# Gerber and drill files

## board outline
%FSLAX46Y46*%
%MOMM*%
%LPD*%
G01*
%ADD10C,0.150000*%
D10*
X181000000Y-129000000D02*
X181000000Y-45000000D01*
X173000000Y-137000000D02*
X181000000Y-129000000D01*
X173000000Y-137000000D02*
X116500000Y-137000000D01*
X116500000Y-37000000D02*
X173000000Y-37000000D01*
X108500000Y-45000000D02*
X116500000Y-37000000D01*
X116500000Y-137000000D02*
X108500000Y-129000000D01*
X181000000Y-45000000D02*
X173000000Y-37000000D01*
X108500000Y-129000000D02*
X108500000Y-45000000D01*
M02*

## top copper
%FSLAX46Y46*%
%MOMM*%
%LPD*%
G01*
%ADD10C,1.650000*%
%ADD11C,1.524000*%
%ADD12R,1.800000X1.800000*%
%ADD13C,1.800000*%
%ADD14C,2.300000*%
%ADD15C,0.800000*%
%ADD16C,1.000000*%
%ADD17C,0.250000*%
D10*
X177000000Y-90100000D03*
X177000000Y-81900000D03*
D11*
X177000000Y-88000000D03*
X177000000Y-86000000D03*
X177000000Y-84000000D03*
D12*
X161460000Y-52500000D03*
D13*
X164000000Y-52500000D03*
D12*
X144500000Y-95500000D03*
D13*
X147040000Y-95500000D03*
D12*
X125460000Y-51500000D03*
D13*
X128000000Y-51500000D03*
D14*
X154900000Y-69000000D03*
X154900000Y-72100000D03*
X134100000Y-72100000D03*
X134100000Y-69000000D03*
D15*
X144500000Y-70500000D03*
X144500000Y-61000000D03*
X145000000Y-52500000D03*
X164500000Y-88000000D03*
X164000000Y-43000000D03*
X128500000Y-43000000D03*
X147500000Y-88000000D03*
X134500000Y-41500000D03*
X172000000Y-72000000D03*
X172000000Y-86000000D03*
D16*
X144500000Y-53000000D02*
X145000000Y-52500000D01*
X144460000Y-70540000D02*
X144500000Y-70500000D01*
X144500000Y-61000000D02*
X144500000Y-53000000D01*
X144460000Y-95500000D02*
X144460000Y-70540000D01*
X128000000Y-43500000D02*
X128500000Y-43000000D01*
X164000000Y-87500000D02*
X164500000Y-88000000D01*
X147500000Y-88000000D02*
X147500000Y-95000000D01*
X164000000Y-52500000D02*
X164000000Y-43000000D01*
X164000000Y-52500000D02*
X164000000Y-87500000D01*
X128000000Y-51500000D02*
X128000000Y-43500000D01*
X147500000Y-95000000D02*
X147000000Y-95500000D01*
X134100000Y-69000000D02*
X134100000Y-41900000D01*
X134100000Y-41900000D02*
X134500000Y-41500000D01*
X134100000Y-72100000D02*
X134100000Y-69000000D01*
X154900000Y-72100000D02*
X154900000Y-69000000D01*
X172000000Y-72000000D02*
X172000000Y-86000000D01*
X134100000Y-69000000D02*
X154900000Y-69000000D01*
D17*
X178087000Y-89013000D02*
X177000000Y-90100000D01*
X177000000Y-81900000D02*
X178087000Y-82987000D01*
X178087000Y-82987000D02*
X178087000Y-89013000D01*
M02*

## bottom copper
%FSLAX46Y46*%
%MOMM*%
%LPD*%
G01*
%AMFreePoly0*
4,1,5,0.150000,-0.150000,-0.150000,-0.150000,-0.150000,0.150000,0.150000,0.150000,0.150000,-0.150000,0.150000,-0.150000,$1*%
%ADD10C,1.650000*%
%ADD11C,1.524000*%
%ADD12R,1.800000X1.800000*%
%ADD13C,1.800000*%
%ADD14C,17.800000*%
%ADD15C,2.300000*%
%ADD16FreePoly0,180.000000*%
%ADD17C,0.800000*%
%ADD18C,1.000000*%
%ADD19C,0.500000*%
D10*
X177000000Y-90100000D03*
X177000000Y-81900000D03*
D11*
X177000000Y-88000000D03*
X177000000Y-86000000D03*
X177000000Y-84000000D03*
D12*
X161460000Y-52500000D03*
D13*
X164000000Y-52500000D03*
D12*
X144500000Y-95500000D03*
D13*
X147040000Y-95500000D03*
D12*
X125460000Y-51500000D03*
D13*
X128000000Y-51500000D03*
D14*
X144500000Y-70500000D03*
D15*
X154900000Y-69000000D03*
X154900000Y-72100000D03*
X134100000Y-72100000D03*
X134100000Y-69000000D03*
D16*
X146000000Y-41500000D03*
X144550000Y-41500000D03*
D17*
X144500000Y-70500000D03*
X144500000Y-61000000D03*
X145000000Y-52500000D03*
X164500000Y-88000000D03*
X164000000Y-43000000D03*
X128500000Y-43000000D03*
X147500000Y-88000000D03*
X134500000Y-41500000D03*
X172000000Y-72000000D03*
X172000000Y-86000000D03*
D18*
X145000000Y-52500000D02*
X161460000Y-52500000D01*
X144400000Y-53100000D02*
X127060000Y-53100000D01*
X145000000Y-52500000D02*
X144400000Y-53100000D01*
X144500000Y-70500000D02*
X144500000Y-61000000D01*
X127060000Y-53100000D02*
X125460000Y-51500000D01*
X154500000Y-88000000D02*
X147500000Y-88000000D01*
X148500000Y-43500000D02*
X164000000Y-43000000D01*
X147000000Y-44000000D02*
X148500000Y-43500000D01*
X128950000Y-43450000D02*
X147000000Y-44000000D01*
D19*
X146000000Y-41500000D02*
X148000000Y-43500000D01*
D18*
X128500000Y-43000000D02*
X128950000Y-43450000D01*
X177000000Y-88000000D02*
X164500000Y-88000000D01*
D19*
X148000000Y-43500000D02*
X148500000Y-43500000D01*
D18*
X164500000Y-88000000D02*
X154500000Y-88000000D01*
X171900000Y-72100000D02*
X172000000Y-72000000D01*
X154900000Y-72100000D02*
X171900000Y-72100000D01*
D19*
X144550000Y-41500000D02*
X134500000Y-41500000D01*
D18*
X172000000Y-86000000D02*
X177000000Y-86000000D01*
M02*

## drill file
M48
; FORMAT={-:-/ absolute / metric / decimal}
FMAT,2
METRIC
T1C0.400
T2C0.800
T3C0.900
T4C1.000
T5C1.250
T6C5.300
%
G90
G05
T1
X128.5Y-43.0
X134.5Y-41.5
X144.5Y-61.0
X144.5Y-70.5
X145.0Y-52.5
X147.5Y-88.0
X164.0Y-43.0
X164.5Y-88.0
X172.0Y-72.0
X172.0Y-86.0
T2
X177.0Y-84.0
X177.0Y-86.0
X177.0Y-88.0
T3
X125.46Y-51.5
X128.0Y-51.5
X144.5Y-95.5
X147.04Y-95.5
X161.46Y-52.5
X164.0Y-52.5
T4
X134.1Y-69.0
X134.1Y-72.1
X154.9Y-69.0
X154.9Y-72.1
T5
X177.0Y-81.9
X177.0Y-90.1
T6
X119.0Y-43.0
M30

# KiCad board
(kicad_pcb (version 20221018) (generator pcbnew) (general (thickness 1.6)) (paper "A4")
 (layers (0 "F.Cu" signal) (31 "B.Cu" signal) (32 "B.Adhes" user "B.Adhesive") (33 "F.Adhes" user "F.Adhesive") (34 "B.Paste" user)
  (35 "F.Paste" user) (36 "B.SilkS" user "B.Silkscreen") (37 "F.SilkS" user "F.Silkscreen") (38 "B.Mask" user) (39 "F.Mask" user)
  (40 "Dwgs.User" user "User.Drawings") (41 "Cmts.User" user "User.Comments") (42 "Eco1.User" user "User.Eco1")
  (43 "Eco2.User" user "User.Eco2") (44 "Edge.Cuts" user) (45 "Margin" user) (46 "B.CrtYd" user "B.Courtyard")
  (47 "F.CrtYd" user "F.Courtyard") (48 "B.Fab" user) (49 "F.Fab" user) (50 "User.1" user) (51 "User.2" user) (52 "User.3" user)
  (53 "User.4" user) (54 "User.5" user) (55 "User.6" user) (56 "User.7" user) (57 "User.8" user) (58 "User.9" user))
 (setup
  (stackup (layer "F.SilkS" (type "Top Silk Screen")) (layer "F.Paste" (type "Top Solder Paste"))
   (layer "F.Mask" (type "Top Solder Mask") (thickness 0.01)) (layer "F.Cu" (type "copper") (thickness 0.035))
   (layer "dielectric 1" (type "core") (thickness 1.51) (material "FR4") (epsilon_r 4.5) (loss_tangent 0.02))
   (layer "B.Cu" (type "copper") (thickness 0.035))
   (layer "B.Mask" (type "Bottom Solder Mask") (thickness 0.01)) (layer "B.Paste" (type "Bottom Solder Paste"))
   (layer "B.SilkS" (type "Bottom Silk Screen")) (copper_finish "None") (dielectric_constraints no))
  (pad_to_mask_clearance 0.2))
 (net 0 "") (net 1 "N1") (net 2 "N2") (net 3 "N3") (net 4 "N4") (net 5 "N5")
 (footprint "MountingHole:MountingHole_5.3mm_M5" (layer "F.Cu") (at 119 43)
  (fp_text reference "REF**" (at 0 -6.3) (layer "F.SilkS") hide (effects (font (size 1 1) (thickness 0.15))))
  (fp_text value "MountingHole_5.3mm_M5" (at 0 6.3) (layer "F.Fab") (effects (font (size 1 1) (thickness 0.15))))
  (pad "" np_thru_hole circle (at 0 0) (size 5.3 5.3) (drill 5.3) (layers "*.Cu" "*.Mask")))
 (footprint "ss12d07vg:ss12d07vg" (layer "F.Cu") (at 177 90.1 90)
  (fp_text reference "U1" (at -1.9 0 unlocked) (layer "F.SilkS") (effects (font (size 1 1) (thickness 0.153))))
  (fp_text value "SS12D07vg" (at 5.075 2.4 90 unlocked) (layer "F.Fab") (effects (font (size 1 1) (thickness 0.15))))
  (pad "1" thru_hole circle (at 0 0 90) (size 1.65 1.65) (drill 1.25) (layers "*.Cu" "*.Mask") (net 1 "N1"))
  (pad "1" thru_hole circle (at 8.2 0 90) (size 1.65 1.65) (drill 1.25) (layers "*.Cu" "*.Mask") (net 1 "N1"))
  (pad "2" thru_hole circle (at 2.1 0 90) (size 1.524 1.524) (drill 0.8) (layers "*.Cu" "*.Mask") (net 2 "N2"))
  (pad "3" thru_hole circle (at 4.1 0 90) (size 1.524 1.524) (drill 0.8) (layers "*.Cu" "*.Mask") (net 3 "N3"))
  (pad "4" thru_hole circle (at 6.1 0 90) (size 1.524 1.524) (drill 0.8) (layers "*.Cu" "*.Mask") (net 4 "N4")))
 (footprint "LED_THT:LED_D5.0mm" (layer "F.Cu") (at 161.46 52.5)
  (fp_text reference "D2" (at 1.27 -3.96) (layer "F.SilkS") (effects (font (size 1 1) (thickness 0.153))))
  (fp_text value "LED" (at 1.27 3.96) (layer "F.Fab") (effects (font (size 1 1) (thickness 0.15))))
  (pad "1" thru_hole rect (at 0 0) (size 1.8 1.8) (drill 0.9) (layers "*.Cu" "*.Mask") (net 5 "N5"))
  (pad "2" thru_hole circle (at 2.54 0) (size 1.8 1.8) (drill 0.9) (layers "*.Cu" "*.Mask") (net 2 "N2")))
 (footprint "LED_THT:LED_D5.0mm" (layer "F.Cu") (at 144.5 95.5)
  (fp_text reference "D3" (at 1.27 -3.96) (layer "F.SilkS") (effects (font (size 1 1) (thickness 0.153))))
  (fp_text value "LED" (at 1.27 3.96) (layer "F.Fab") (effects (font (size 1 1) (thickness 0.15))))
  (pad "1" thru_hole rect (at 0 0) (size 1.8 1.8) (drill 0.9) (layers "*.Cu" "*.Mask") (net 5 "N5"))
  (pad "2" thru_hole circle (at 2.54 0) (size 1.8 1.8) (drill 0.9) (layers "*.Cu" "*.Mask") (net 2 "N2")))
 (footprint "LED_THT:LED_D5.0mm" (layer "F.Cu") (at 125.46 51.5)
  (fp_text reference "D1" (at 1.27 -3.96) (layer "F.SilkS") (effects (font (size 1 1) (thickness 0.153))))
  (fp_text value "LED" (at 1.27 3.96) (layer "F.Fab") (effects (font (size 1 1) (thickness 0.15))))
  (pad "1" thru_hole rect (at 0 0) (size 1.8 1.8) (drill 0.9) (layers "*.Cu" "*.Mask") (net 5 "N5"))
  (pad "2" thru_hole circle (at 2.54 0) (size 1.8 1.8) (drill 0.9) (layers "*.Cu" "*.Mask") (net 2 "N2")))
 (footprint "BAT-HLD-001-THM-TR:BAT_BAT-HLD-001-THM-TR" (layer "B.Cu") (at 144.5 70.5 180)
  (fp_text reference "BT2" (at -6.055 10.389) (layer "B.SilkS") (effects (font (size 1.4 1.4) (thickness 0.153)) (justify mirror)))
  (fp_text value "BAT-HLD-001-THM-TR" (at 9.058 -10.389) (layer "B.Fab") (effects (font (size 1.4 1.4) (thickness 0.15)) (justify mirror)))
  (pad "N" smd circle (at 0 0 180) (size 17.8 17.8) (layers "B.Cu" "B.Mask") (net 5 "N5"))
  (pad "P1" thru_hole circle (at -10.4 1.5 180) (size 2.3 2.3) (drill 1) (layers "*.Cu" "*.Mask") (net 3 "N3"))
  (pad "P2" thru_hole circle (at -10.4 -1.6 180) (size 2.3 2.3) (drill 1) (layers "*.Cu" "*.Mask") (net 3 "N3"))
  (pad "P3" thru_hole circle (at 10.4 -1.6 180) (size 2.3 2.3) (drill 1) (layers "*.Cu" "*.Mask") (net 3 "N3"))
  (pad "P4" thru_hole circle (at 10.4 1.5 180) (size 2.3 2.3) (drill 1) (layers "*.Cu" "*.Mask") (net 3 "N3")))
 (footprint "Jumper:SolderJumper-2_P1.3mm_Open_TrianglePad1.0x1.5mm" (layer "B.Cu") (at 145.275 41.5 180)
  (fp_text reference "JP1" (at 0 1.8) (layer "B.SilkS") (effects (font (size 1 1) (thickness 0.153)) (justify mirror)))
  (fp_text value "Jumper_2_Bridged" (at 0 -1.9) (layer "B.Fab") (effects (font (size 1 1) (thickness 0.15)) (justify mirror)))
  (pad "1" smd custom (at -0.725 0 180) (size 0.3 0.3) (layers "B.Cu" "B.Mask") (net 2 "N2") (zone_connect 2) (thermal_bridge_angle 45)
   (options (clearance outline) (anchor rect)) (primitives))
  (pad "2" smd custom (at 0.725 0 180) (size 0.3 0.3) (layers "B.Cu" "B.Mask") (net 3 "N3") (zone_connect 2) (thermal_bridge_angle 45)
   (options (clearance outline) (anchor rect)) (primitives)))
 (gr_line (start 181 129) (end 181 45) (stroke (width 0.15) (type default)) (layer "Edge.Cuts"))
 (gr_line (start 173 137) (end 181 129) (stroke (width 0.15) (type default)) (layer "Edge.Cuts"))
 (gr_line (start 173 137) (end 116.5 137) (stroke (width 0.15) (type default)) (layer "Edge.Cuts"))
 (gr_line (start 116.5 37) (end 173 37) (stroke (width 0.15) (type default)) (layer "Edge.Cuts"))
 (gr_line (start 108.5 45) (end 116.5 37) (stroke (width 0.15) (type default)) (layer "Edge.Cuts"))
 (gr_line (start 116.5 137) (end 108.5 129) (stroke (width 0.15) (type default)) (layer "Edge.Cuts"))
 (gr_line (start 181 45) (end 173 37) (stroke (width 0.15) (type default)) (layer "Edge.Cuts"))
 (gr_line (start 108.5 129) (end 108.5 45) (stroke (width 0.15) (type default)) (layer "Edge.Cuts"))
 (segment (start 144.5 53) (end 145 52.5) (width 1) (layer "F.Cu") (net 5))
 (segment (start 144.46 70.54) (end 144.5 70.5) (width 1) (layer "F.Cu") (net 5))
 (segment (start 144.5 61) (end 144.5 53) (width 1) (layer "F.Cu") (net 5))
 (segment (start 144.46 95.5) (end 144.46 70.54) (width 1) (layer "F.Cu") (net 5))
 (via (at 144.5 70.5) (size 0.8) (drill 0.4) (layers "F.Cu" "B.Cu") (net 5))
 (via (at 144.5 61) (size 0.8) (drill 0.4) (layers "F.Cu" "B.Cu") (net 5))
 (via (at 145 52.5) (size 0.8) (drill 0.4) (layers "F.Cu" "B.Cu") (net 5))
 (segment (start 145 52.5) (end 161.46 52.5) (width 1) (layer "B.Cu") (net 5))
 (segment (start 144.4 53.1) (end 127.06 53.1) (width 1) (layer "B.Cu") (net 5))
 (segment (start 145 52.5) (end 144.4 53.1) (width 1) (layer "B.Cu") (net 5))
 (segment (start 144.5 70.5) (end 144.5 61) (width 1) (layer "B.Cu") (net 5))
 (segment (start 127.06 53.1) (end 125.46 51.5) (width 1) (layer "B.Cu") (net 5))
 (segment (start 128 43.5) (end 128.5 43) (width 1) (layer "F.Cu") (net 2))
 (segment (start 164 87.5) (end 164.5 88) (width 1) (layer "F.Cu") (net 2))
 (segment (start 147.5 88) (end 147.5 95) (width 1) (layer "F.Cu") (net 2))
 (segment (start 164 52.5) (end 164 43) (width 1) (layer "F.Cu") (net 2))
 (segment (start 164 52.5) (end 164 87.5) (width 1) (layer "F.Cu") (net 2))
 (segment (start 128 51.5) (end 128 43.5) (width 1) (layer "F.Cu") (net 2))
 (segment (start 147.5 95) (end 147 95.5) (width 1) (layer "F.Cu") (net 2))
 (via (at 164.5 88) (size 0.8) (drill 0.4) (layers "F.Cu" "B.Cu") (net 2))
 (via (at 164 43) (size 0.8) (drill 0.4) (layers "F.Cu" "B.Cu") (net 2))
 (via (at 128.5 43) (size 0.8) (drill 0.4) (layers "F.Cu" "B.Cu") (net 2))
 (via (at 147.5 88) (size 0.8) (drill 0.4) (layers "F.Cu" "B.Cu") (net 2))
 (segment (start 154.5 88) (end 147.5 88) (width 1) (layer "B.Cu") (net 2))
 (segment (start 148.5 43.5) (end 164 43) (width 1) (layer "B.Cu") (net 2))
 (segment (start 147 44) (end 148.5 43.5) (width 1) (layer "B.Cu") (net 2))
 (segment (start 128.95 43.45) (end 147 44) (width 1) (layer "B.Cu") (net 2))
 (segment (start 146 41.5) (end 148 43.5) (width 0.5) (layer "B.Cu") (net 2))
 (segment (start 128.5 43) (end 128.95 43.45) (width 1) (layer "B.Cu") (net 2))
 (segment (start 177 88) (end 164.5 88) (width 1) (layer "B.Cu") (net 2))
 (segment (start 148 43.5) (end 148.5 43.5) (width 0.5) (layer "B.Cu") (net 2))
 (segment (start 164.5 88) (end 154.5 88) (width 1) (layer "B.Cu") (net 2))
 (segment (start 134.1 69) (end 134.1 41.9) (width 1) (layer "F.Cu") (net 3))
 (segment (start 134.1 41.9) (end 134.5 41.5) (width 1) (layer "F.Cu") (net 3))
 (segment (start 134.1 72.1) (end 134.1 69) (width 1) (layer "F.Cu") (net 3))
 (segment (start 154.9 72.1) (end 154.9 69) (width 1) (layer "F.Cu") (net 3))
 (segment (start 172 72) (end 172 86) (width 1) (layer "F.Cu") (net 3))
 (segment (start 134.1 69) (end 154.9 69) (width 1) (layer "F.Cu") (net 3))
 (via (at 134.5 41.5) (size 0.8) (drill 0.4) (layers "F.Cu" "B.Cu") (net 3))
 (via (at 172 72) (size 0.8) (drill 0.4) (layers "F.Cu" "B.Cu") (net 3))
 (via (at 172 86) (size 0.8) (drill 0.4) (layers "F.Cu" "B.Cu") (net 3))
 (segment (start 171.9 72.1) (end 172 72) (width 1) (layer "B.Cu") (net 3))
 (segment (start 154.9 72.1) (end 171.9 72.1) (width 1) (layer "B.Cu") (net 3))
 (segment (start 144.55 41.5) (end 134.5 41.5) (width 0.5) (layer "B.Cu") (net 3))
 (segment (start 172 86) (end 177 86) (width 1) (layer "B.Cu") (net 3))
 (segment (start 178.087 89.013) (end 177 90.1) (width 0.25) (layer "F.Cu") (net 1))
 (segment (start 177 81.9) (end 178.087 82.987) (width 0.25) (layer "F.Cu") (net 1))
 (segment (start 178.087 82.987) (end 178.087 89.013) (width 0.25) (layer "F.Cu") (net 1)))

